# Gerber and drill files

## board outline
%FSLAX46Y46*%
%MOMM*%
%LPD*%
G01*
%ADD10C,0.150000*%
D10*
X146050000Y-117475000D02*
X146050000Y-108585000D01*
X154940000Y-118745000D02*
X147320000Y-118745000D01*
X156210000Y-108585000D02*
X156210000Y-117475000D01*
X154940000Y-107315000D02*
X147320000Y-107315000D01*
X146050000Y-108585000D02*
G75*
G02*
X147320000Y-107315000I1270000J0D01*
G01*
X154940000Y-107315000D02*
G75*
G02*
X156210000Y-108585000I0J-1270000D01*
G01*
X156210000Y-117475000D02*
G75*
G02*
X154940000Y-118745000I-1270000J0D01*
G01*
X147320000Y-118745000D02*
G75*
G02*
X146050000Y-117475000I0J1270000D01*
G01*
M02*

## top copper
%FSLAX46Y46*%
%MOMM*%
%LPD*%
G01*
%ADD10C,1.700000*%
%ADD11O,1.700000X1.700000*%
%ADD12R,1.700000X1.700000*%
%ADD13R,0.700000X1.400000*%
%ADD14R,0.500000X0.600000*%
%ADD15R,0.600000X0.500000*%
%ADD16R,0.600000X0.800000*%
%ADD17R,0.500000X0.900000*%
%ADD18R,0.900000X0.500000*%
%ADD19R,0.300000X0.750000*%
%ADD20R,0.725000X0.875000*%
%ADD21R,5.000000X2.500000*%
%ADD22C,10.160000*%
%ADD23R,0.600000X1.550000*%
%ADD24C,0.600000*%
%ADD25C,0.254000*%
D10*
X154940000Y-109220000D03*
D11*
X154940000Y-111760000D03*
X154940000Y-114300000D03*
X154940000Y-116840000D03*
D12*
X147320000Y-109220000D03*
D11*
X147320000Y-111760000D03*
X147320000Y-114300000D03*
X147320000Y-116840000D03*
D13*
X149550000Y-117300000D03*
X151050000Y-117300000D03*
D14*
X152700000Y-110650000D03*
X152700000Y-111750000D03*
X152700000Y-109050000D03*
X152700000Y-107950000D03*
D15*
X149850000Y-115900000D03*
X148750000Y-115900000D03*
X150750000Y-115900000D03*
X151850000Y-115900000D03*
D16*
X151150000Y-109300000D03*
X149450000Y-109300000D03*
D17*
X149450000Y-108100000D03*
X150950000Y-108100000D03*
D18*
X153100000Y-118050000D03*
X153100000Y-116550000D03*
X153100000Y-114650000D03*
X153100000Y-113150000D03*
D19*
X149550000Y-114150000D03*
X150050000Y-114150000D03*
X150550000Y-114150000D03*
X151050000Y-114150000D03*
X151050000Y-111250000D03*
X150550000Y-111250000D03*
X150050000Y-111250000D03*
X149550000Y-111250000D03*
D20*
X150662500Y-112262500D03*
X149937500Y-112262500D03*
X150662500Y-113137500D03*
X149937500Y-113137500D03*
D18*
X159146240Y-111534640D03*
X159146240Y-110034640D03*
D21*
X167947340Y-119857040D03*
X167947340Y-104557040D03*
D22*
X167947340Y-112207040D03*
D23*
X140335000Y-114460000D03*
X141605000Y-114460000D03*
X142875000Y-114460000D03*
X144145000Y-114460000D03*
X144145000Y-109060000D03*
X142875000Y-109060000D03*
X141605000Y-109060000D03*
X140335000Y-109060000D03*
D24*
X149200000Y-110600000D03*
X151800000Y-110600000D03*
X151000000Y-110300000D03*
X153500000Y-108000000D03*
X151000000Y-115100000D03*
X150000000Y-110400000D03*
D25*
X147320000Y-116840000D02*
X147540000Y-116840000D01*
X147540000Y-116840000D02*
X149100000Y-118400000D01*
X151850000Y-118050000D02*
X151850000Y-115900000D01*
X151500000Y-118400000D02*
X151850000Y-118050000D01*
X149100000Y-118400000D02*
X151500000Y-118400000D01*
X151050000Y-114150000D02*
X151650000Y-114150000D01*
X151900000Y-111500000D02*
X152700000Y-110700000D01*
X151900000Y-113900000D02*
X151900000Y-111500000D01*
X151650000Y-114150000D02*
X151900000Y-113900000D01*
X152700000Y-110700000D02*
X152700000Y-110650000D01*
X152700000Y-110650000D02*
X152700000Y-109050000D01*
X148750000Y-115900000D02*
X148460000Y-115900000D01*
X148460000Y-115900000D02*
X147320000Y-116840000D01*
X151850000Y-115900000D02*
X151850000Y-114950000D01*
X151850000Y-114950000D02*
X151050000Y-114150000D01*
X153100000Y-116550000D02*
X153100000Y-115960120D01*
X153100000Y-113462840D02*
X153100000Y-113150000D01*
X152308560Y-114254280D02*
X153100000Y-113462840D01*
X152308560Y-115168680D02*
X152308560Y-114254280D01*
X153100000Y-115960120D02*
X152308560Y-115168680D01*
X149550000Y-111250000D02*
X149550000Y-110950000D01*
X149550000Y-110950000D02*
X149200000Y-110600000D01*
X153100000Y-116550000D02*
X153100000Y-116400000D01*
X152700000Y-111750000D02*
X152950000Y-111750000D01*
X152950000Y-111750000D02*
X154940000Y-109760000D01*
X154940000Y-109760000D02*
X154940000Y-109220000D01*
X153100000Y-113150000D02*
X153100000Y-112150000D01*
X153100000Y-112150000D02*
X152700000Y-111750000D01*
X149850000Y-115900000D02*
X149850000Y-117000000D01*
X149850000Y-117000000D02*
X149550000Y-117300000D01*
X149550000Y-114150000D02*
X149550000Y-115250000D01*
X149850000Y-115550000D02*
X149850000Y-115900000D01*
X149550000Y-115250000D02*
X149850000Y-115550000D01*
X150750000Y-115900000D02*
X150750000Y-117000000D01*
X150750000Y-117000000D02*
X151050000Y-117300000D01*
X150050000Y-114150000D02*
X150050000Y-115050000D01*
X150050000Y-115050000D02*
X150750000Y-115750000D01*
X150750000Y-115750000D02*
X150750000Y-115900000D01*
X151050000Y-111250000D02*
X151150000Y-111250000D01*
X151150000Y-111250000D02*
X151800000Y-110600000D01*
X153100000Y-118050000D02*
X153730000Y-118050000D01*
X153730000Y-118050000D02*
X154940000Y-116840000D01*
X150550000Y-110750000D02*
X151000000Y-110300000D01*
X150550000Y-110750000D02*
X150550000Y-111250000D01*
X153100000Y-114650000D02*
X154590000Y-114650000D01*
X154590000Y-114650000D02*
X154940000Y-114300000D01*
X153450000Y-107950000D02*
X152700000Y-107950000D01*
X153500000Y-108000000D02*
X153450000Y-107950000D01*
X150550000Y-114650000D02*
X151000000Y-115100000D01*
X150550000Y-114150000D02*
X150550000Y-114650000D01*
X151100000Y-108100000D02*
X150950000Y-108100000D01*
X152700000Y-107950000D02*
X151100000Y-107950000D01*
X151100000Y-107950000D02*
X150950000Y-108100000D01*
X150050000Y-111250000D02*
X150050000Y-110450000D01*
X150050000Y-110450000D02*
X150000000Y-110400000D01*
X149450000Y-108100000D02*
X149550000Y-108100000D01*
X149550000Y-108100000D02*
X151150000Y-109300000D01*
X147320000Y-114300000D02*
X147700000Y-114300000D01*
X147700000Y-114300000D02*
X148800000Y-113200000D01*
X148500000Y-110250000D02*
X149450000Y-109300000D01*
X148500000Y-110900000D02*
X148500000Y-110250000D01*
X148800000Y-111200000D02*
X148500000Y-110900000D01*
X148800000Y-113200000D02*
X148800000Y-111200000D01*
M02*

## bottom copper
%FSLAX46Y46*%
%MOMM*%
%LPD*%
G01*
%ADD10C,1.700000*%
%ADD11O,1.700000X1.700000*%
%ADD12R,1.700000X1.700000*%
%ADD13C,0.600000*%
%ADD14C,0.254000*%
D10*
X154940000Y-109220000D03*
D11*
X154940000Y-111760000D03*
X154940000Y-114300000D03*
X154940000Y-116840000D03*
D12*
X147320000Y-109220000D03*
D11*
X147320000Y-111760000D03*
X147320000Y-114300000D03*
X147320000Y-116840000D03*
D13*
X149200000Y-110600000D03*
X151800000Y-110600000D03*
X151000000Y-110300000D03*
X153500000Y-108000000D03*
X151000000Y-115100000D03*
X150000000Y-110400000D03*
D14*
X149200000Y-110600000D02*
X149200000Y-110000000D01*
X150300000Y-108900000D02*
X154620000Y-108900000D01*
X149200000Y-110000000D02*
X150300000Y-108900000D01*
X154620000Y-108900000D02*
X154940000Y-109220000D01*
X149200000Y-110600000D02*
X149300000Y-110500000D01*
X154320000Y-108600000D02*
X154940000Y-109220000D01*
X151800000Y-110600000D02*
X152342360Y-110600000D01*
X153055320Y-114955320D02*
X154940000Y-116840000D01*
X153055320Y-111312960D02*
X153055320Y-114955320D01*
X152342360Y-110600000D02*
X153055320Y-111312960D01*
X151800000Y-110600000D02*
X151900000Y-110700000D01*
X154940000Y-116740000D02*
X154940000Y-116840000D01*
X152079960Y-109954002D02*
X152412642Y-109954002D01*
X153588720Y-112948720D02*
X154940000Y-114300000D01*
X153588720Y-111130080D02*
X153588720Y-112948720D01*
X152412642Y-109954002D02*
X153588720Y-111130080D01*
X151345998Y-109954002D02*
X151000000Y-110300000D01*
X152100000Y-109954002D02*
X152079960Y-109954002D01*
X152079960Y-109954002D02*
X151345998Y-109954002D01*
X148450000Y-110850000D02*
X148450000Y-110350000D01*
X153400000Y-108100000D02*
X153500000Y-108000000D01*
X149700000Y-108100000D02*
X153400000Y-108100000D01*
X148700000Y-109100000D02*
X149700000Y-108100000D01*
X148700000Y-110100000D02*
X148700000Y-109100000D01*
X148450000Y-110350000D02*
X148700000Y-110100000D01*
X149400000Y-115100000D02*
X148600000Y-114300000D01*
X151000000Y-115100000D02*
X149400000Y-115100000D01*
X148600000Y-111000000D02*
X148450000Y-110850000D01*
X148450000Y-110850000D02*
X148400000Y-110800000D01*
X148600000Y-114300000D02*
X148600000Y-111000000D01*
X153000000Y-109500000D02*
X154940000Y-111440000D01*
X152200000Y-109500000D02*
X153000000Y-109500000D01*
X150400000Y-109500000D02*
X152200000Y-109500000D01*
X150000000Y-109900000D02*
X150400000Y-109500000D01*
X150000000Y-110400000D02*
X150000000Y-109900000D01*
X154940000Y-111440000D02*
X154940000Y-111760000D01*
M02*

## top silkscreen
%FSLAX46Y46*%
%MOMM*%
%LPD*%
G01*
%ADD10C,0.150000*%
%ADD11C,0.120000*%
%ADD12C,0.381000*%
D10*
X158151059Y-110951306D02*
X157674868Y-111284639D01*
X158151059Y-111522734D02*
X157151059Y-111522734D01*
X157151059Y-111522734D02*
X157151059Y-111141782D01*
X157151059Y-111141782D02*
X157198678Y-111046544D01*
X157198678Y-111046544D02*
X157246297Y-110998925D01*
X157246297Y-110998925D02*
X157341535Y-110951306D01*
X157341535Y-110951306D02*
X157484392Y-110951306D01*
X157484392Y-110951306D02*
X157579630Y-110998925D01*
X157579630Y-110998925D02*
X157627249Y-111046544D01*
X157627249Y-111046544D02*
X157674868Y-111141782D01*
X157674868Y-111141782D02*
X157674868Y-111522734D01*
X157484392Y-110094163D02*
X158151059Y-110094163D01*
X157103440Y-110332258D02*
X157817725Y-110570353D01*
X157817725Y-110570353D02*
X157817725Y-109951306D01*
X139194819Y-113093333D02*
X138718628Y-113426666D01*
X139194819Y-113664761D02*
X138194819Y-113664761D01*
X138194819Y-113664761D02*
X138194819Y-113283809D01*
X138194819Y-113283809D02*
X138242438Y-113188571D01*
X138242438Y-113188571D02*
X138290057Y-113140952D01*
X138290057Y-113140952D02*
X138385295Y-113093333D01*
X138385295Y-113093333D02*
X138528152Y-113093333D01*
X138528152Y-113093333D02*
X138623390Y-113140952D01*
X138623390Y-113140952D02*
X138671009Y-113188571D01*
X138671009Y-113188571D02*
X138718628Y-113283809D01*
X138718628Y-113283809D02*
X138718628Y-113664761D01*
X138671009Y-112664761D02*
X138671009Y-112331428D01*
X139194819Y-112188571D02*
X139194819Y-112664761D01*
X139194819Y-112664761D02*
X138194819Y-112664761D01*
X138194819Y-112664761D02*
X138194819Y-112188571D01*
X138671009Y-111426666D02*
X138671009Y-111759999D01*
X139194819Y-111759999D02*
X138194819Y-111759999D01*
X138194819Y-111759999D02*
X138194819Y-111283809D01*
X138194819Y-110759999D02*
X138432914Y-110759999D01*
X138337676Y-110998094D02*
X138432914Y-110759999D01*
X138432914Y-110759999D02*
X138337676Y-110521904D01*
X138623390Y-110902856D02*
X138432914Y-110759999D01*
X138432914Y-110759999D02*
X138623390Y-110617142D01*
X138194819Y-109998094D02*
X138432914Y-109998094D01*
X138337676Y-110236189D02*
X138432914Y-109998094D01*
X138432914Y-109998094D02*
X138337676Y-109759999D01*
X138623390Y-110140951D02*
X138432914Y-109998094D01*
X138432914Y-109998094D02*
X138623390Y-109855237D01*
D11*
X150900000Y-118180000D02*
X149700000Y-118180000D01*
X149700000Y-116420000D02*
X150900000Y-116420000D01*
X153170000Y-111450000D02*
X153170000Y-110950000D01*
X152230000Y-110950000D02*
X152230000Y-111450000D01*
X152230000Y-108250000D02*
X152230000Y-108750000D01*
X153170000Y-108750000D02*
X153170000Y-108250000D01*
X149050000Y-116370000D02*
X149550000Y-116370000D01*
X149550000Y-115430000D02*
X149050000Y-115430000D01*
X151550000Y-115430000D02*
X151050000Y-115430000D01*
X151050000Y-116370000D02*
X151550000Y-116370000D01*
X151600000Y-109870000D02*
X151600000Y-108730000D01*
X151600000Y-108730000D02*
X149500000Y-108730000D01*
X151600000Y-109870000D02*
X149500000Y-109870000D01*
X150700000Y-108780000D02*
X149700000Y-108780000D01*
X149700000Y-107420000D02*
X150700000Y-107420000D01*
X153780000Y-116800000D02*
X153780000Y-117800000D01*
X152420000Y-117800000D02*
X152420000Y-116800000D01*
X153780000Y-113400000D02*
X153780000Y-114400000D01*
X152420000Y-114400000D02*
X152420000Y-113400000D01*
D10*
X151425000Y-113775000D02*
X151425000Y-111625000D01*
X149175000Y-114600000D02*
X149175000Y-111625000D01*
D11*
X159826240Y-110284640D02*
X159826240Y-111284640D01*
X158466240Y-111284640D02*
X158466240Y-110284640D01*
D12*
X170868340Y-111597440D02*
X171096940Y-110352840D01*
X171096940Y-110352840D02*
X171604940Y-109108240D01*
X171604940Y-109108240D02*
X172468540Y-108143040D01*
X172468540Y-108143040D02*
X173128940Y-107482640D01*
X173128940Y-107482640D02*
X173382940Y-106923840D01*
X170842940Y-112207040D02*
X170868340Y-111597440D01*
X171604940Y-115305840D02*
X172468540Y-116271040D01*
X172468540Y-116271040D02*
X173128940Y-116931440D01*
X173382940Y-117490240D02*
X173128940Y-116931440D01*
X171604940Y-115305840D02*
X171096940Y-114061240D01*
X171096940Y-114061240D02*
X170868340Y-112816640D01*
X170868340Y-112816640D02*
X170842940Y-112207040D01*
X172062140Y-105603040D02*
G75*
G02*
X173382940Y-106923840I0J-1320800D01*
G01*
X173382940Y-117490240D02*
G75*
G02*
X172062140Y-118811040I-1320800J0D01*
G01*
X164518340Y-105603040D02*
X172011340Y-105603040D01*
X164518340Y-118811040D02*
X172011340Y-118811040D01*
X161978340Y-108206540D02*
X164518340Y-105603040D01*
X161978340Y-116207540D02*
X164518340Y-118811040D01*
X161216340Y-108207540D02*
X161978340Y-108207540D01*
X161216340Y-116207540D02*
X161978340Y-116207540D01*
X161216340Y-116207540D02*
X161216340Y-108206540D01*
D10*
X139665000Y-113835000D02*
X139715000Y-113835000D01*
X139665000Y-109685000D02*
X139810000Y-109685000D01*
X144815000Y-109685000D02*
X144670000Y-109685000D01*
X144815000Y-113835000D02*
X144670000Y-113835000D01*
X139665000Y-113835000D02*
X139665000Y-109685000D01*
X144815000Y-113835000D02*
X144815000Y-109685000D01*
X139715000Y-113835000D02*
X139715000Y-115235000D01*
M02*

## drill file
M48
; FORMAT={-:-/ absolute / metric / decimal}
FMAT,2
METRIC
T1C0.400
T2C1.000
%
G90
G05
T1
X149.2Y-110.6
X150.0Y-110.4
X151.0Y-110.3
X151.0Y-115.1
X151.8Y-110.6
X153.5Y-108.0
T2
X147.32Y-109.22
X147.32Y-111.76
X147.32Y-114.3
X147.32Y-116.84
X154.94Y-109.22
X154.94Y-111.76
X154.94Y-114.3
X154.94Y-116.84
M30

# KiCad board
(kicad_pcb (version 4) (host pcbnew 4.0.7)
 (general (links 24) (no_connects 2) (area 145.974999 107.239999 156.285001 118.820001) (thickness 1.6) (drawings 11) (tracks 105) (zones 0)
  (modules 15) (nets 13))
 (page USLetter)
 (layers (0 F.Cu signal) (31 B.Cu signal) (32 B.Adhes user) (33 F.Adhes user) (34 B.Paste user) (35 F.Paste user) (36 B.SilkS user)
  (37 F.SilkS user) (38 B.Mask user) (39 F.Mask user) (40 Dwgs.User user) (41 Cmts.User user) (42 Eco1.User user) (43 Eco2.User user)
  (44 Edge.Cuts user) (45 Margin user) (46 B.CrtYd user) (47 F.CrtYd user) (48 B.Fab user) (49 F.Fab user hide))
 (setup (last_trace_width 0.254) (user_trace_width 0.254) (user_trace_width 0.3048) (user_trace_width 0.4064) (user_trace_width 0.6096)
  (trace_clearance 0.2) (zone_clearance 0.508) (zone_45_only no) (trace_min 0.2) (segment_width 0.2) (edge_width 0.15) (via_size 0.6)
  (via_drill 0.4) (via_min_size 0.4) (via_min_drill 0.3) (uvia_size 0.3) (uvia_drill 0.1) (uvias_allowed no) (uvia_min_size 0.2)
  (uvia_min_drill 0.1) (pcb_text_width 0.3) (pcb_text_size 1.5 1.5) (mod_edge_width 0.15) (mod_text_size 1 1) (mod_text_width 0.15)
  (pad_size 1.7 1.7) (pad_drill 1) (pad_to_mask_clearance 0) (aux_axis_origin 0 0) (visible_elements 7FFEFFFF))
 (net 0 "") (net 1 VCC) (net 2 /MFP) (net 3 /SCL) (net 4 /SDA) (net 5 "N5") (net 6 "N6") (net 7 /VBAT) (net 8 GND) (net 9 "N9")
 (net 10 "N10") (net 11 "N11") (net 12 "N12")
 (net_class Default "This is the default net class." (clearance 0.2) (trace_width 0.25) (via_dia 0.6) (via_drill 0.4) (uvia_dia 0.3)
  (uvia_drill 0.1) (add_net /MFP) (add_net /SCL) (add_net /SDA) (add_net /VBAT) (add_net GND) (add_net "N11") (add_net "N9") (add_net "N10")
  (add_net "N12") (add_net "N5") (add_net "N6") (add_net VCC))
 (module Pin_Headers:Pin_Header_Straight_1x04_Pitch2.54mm (layer F.Cu) (at 154.94 109.22)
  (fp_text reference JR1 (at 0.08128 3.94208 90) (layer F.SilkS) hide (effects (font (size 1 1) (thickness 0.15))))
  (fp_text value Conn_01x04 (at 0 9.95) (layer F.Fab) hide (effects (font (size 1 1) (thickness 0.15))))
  (pad 1 thru_hole circle (at 0 0) (size 1.7 1.7) (drill 1) (layers *.Cu *.Mask) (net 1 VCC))
  (pad 2 thru_hole oval (at 0 2.54) (size 1.7 1.7) (drill 1) (layers *.Cu *.Mask) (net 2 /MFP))
  (pad 3 thru_hole oval (at 0 5.08) (size 1.7 1.7) (drill 1) (layers *.Cu *.Mask) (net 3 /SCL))
  (pad 4 thru_hole oval (at 0 7.62) (size 1.7 1.7) (drill 1) (layers *.Cu *.Mask) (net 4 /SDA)))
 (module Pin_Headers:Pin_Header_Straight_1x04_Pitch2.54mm (layer F.Cu) (at 147.32 109.22)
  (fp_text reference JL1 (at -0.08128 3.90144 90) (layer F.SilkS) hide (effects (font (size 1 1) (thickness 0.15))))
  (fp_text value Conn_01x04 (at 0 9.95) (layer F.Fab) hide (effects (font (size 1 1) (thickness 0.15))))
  (pad 1 thru_hole rect (at 0 0) (size 1.7 1.7) (drill 1) (layers *.Cu *.Mask) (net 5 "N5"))
  (pad 2 thru_hole oval (at 0 2.54) (size 1.7 1.7) (drill 1) (layers *.Cu *.Mask) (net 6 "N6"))
  (pad 3 thru_hole oval (at 0 5.08) (size 1.7 1.7) (drill 1) (layers *.Cu *.Mask) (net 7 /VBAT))
  (pad 4 thru_hole oval (at 0 7.62) (size 1.7 1.7) (drill 1) (layers *.Cu *.Mask) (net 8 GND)))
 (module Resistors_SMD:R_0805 (layer F.Cu) (at 150.3 117.3)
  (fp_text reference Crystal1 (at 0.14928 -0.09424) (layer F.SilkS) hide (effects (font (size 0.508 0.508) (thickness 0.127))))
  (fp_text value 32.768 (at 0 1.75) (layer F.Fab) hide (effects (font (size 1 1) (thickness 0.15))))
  (fp_line (start 0.6 0.88) (end -0.6 0.88) (layer F.SilkS) (width 0.12))
  (fp_line (start -0.6 -0.88) (end 0.6 -0.88) (layer F.SilkS) (width 0.12))
  (pad 1 smd rect (at -0.75 0) (size 0.7 1.4) (layers F.Cu F.Paste F.Mask) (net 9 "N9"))
  (pad 2 smd rect (at 0.75 0) (size 0.7 1.4) (layers F.Cu F.Paste F.Mask) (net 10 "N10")))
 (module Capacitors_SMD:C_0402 (layer F.Cu) (at 152.7 111.2 270)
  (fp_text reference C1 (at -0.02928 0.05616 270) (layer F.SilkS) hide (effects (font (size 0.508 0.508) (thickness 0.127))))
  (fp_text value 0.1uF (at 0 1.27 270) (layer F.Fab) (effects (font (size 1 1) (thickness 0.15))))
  (fp_line (start 0.25 -0.47) (end -0.25 -0.47) (layer F.SilkS) (width 0.12))
  (fp_line (start -0.25 0.47) (end 0.25 0.47) (layer F.SilkS) (width 0.12))
  (pad 1 smd rect (at -0.55 0 270) (size 0.6 0.5) (layers F.Cu F.Paste F.Mask) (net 8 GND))
  (pad 2 smd rect (at 0.55 0 270) (size 0.6 0.5) (layers F.Cu F.Paste F.Mask) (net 1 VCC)))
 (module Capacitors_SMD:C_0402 (layer F.Cu) (at 152.7 108.5 90)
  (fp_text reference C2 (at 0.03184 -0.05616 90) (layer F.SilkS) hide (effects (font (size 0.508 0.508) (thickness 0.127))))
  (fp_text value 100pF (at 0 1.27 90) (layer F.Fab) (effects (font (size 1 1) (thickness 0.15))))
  (fp_line (start 0.25 -0.47) (end -0.25 -0.47) (layer F.SilkS) (width 0.12))
  (fp_line (start -0.25 0.47) (end 0.25 0.47) (layer F.SilkS) (width 0.12))
  (pad 1 smd rect (at -0.55 0 90) (size 0.6 0.5) (layers F.Cu F.Paste F.Mask) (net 8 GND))
  (pad 2 smd rect (at 0.55 0 90) (size 0.6 0.5) (layers F.Cu F.Paste F.Mask) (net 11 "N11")))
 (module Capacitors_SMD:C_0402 (layer F.Cu) (at 149.3 115.9 180)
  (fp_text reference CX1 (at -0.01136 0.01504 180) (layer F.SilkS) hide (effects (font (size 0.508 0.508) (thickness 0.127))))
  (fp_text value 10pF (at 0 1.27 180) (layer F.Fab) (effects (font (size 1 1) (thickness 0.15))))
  (fp_line (start 0.25 -0.47) (end -0.25 -0.47) (layer F.SilkS) (width 0.12))
  (fp_line (start -0.25 0.47) (end 0.25 0.47) (layer F.SilkS) (width 0.12))
  (pad 1 smd rect (at -0.55 0 180) (size 0.6 0.5) (layers F.Cu F.Paste F.Mask) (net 9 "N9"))
  (pad 2 smd rect (at 0.55 0 180) (size 0.6 0.5) (layers F.Cu F.Paste F.Mask) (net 8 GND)))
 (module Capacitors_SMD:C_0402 (layer F.Cu) (at 151.3 115.9)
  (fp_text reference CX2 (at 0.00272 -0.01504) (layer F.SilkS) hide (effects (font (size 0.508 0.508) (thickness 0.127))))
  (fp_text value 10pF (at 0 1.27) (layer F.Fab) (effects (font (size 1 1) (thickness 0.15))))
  (fp_line (start 0.25 -0.47) (end -0.25 -0.47) (layer F.SilkS) (width 0.12))
  (fp_line (start -0.25 0.47) (end 0.25 0.47) (layer F.SilkS) (width 0.12))
  (pad 1 smd rect (at -0.55 0) (size 0.6 0.5) (layers F.Cu F.Paste F.Mask) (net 10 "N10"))
  (pad 2 smd rect (at 0.55 0) (size 0.6 0.5) (layers F.Cu F.Paste F.Mask) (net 8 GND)))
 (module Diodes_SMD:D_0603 (layer F.Cu) (at 150.3 109.3 180)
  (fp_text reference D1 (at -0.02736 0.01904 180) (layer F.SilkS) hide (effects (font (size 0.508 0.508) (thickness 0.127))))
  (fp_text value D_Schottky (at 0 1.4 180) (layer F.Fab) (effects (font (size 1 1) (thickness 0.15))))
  (fp_line (start -1.3 -0.57) (end -1.3 0.57) (layer F.SilkS) (width 0.12))
  (fp_line (start -1.3 0.57) (end 0.8 0.57) (layer F.SilkS) (width 0.12))
  (fp_line (start -1.3 -0.57) (end 0.8 -0.57) (layer F.SilkS) (width 0.12))
  (pad 1 smd rect (at -0.85 0 180) (size 0.6 0.8) (layers F.Cu F.Paste F.Mask) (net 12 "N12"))
  (pad 2 smd rect (at 0.85 0 180) (size 0.6 0.8) (layers F.Cu F.Paste F.Mask) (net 7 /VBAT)))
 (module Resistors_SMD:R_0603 (layer F.Cu) (at 150.2 108.1)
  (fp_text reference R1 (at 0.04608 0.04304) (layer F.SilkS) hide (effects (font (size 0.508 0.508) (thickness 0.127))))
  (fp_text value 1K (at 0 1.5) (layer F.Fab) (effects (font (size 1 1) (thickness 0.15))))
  (fp_line (start 0.5 0.68) (end -0.5 0.68) (layer F.SilkS) (width 0.12))
  (fp_line (start -0.5 -0.68) (end 0.5 -0.68) (layer F.SilkS) (width 0.12))
  (pad 1 smd rect (at -0.75 0) (size 0.5 0.9) (layers F.Cu F.Paste F.Mask) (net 12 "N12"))
  (pad 2 smd rect (at 0.75 0) (size 0.5 0.9) (layers F.Cu F.Paste F.Mask) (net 11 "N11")))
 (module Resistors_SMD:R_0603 (layer F.Cu) (at 153.1 117.3 90)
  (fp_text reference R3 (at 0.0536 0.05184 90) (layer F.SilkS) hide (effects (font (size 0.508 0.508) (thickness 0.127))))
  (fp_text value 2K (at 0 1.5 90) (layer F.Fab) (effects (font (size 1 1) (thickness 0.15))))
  (fp_line (start 0.5 0.68) (end -0.5 0.68) (layer F.SilkS) (width 0.12))
  (fp_line (start -0.5 -0.68) (end 0.5 -0.68) (layer F.SilkS) (width 0.12))
  (pad 1 smd rect (at -0.75 0 90) (size 0.5 0.9) (layers F.Cu F.Paste F.Mask) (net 4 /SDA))
  (pad 2 smd rect (at 0.75 0 90) (size 0.5 0.9) (layers F.Cu F.Paste F.Mask) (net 1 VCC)))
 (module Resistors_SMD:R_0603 (layer F.Cu) (at 153.1 113.9 90)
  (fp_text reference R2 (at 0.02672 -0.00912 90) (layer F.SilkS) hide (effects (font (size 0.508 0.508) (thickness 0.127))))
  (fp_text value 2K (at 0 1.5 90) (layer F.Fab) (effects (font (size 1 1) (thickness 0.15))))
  (fp_line (start 0.5 0.68) (end -0.5 0.68) (layer F.SilkS) (width 0.12))
  (fp_line (start -0.5 -0.68) (end 0.5 -0.68) (layer F.SilkS) (width 0.12))
  (pad 1 smd rect (at -0.75 0 90) (size 0.5 0.9) (layers F.Cu F.Paste F.Mask) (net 3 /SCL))
  (pad 2 smd rect (at 0.75 0 90) (size 0.5 0.9) (layers F.Cu F.Paste F.Mask) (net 1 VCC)))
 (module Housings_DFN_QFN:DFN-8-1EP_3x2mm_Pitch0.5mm (layer F.Cu) (at 150.3 112.7 90)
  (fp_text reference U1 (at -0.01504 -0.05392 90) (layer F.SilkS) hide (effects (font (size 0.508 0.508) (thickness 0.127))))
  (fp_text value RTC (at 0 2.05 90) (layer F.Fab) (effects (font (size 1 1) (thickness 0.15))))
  (fp_line (start -1.075 1.125) (end 1.075 1.125) (layer F.SilkS) (width 0.15))
  (fp_line (start -1.9 -1.125) (end 1.075 -1.125) (layer F.SilkS) (width 0.15))
  (pad 1 smd rect (at -1.45 -0.75 90) (size 0.75 0.3) (layers F.Cu F.Paste F.Mask) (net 9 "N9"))
  (pad 2 smd rect (at -1.45 -0.25 90) (size 0.75 0.3) (layers F.Cu F.Paste F.Mask) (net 10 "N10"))
  (pad 3 smd rect (at -1.45 0.25 90) (size 0.75 0.3) (layers F.Cu F.Paste F.Mask) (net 11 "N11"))
  (pad 4 smd rect (at -1.45 0.75 90) (size 0.75 0.3) (layers F.Cu F.Paste F.Mask) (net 8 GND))
  (pad 5 smd rect (at 1.45 0.75 90) (size 0.75 0.3) (layers F.Cu F.Paste F.Mask) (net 4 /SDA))
  (pad 6 smd rect (at 1.45 0.25 90) (size 0.75 0.3) (layers F.Cu F.Paste F.Mask) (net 3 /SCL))
  (pad 7 smd rect (at 1.45 -0.25 90) (size 0.75 0.3) (layers F.Cu F.Paste F.Mask) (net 2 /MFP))
  (pad 8 smd rect (at 1.45 -0.75 90) (size 0.75 0.3) (layers F.Cu F.Paste F.Mask) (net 1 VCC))
  (pad 9 smd rect (at 0.4375 0.3625 90) (size 0.875 0.725) (layers F.Cu F.Paste F.Mask) (solder_paste_margin_ratio -0.2))
  (pad 9 smd rect (at 0.4375 -0.3625 90) (size 0.875 0.725) (layers F.Cu F.Paste F.Mask) (solder_paste_margin_ratio -0.2))
  (pad 9 smd rect (at -0.4375 0.3625 90) (size 0.875 0.725) (layers F.Cu F.Paste F.Mask) (solder_paste_margin_ratio -0.2))
  (pad 9 smd rect (at -0.4375 -0.3625 90) (size 0.875 0.725) (layers F.Cu F.Paste F.Mask) (solder_paste_margin_ratio -0.2)))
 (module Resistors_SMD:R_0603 (layer F.Cu) (at 159.14624 110.78464 90)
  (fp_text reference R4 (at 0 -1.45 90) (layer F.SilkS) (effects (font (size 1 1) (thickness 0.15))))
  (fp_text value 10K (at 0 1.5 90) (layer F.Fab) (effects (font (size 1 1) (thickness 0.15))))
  (fp_line (start 0.5 0.68) (end -0.5 0.68) (layer F.SilkS) (width 0.12))
  (fp_line (start -0.5 -0.68) (end 0.5 -0.68) (layer F.SilkS) (width 0.12))
  (pad 1 smd rect (at -0.75 0 90) (size 0.5 0.9) (layers F.Cu F.Paste F.Mask) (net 2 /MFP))
  (pad 2 smd rect (at 0.75 0 90) (size 0.5 0.9) (layers F.Cu F.Paste F.Mask) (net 1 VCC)))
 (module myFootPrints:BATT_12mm (layer F.Cu) (at 167.94734 112.20704 90)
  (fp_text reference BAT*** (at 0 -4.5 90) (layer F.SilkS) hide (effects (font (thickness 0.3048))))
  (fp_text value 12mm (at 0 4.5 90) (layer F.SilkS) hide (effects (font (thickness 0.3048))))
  (fp_line (start 0.6096 2.921) (end 1.8542 3.1496) (layer F.SilkS) (width 0.381))
  (fp_line (start 1.8542 3.1496) (end 3.0988 3.6576) (layer F.SilkS) (width 0.381))
  (fp_line (start 3.0988 3.6576) (end 4.064 4.5212) (layer F.SilkS) (width 0.381))
  (fp_line (start 4.064 4.5212) (end 4.7244 5.1816) (layer F.SilkS) (width 0.381))
  (fp_line (start 4.7244 5.1816) (end 5.2832 5.4356) (layer F.SilkS) (width 0.381))
  (fp_line (start 0 2.8956) (end 0.6096 2.921) (layer F.SilkS) (width 0.381))
  (fp_line (start -3.0988 3.6576) (end -4.064 4.5212) (layer F.SilkS) (width 0.381))
  (fp_line (start -4.064 4.5212) (end -4.7244 5.1816) (layer F.SilkS) (width 0.381))
  (fp_line (start -5.2832 5.4356) (end -4.7244 5.1816) (layer F.SilkS) (width 0.381))
  (fp_line (start -3.0988 3.6576) (end -1.8542 3.1496) (layer F.SilkS) (width 0.381))
  (fp_line (start -1.8542 3.1496) (end -0.6096 2.921) (layer F.SilkS) (width 0.381))
  (fp_line (start -0.6096 2.921) (end 0 2.8956) (layer F.SilkS) (width 0.381))
  (fp_arc (start 5.2832 4.1148) (end 6.604 4.1148) (angle 90) (layer F.SilkS) (width 0.381))
  (fp_arc (start -5.2832 4.1148) (end -5.2832 5.4356) (angle 90) (layer F.SilkS) (width 0.381))
  (fp_line (start 6.604 -3.429) (end 6.604 4.064) (layer F.SilkS) (width 0.381))
  (fp_line (start -6.604 -3.429) (end -6.604 4.064) (layer F.SilkS) (width 0.381))
  (fp_line (start 4.0005 -5.969) (end 6.604 -3.429) (layer F.SilkS) (width 0.381))
  (fp_line (start -4.0005 -5.969) (end -6.604 -3.429) (layer F.SilkS) (width 0.381))
  (fp_line (start 3.9995 -6.731) (end 3.9995 -5.969) (layer F.SilkS) (width 0.381))
  (fp_line (start -4.0005 -6.731) (end -4.0005 -5.969) (layer F.SilkS) (width 0.381))
  (fp_line (start -4.0005 -6.731) (end 4.0005 -6.731) (layer F.SilkS) (width 0.381))
  (pad 1 smd rect (at -7.65 0 90) (size 2.5 5) (layers F.Cu F.Paste F.Mask))
  (pad 1 smd rect (at 7.65 0 90) (size 2.5 5) (layers F.Cu F.Paste F.Mask))
  (pad 2 smd circle (at 0 0 90) (size 10.16 10.16) (layers F.Cu F.Paste F.Mask)))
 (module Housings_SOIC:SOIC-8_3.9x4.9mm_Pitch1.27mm (layer F.Cu) (at 142.24 111.76 90)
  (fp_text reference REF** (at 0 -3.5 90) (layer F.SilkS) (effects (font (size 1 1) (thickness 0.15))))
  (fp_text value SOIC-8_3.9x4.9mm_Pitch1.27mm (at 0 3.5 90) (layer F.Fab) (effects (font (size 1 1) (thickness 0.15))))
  (fp_line (start -2.075 -2.575) (end -2.075 -2.525) (layer F.SilkS) (width 0.15))
  (fp_line (start 2.075 -2.575) (end 2.075 -2.43) (layer F.SilkS) (width 0.15))
  (fp_line (start 2.075 2.575) (end 2.075 2.43) (layer F.SilkS) (width 0.15))
  (fp_line (start -2.075 2.575) (end -2.075 2.43) (layer F.SilkS) (width 0.15))
  (fp_line (start -2.075 -2.575) (end 2.075 -2.575) (layer F.SilkS) (width 0.15))
  (fp_line (start -2.075 2.575) (end 2.075 2.575) (layer F.SilkS) (width 0.15))
  (fp_line (start -2.075 -2.525) (end -3.475 -2.525) (layer F.SilkS) (width 0.15))
  (pad 1 smd rect (at -2.7 -1.905 90) (size 1.55 0.6) (layers F.Cu F.Paste F.Mask))
  (pad 2 smd rect (at -2.7 -0.635 90) (size 1.55 0.6) (layers F.Cu F.Paste F.Mask))
  (pad 3 smd rect (at -2.7 0.635 90) (size 1.55 0.6) (layers F.Cu F.Paste F.Mask))
  (pad 4 smd rect (at -2.7 1.905 90) (size 1.55 0.6) (layers F.Cu F.Paste F.Mask))
  (pad 5 smd rect (at 2.7 1.905 90) (size 1.55 0.6) (layers F.Cu F.Paste F.Mask))
  (pad 6 smd rect (at 2.7 0.635 90) (size 1.55 0.6) (layers F.Cu F.Paste F.Mask))
  (pad 7 smd rect (at 2.7 -0.635 90) (size 1.55 0.6) (layers F.Cu F.Paste F.Mask))
  (pad 8 smd rect (at 2.7 -1.905 90) (size 1.55 0.6) (layers F.Cu F.Paste F.Mask)))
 (gr_line (start 146.05 117.475) (end 146.05 108.585) (angle 90) (layer Edge.Cuts) (width 0.15))
 (gr_line (start 154.94 118.745) (end 147.32 118.745) (angle 90) (layer Edge.Cuts) (width 0.15))
 (gr_line (start 156.21 108.585) (end 156.21 117.475) (angle 90) (layer Edge.Cuts) (width 0.15))
 (gr_line (start 154.94 107.315) (end 147.32 107.315) (angle 90) (layer Edge.Cuts) (width 0.15))
 (gr_arc (start 147.32 108.585) (end 146.05 108.585) (angle 90) (layer Edge.Cuts) (width 0.15))
 (gr_arc (start 154.94 108.585) (end 154.94 107.315) (angle 90) (layer Edge.Cuts) (width 0.15))
 (gr_arc (start 154.94 117.475) (end 156.21 117.475) (angle 90) (layer Edge.Cuts) (width 0.15))
 (gr_arc (start 147.32 117.475) (end 147.32 118.745) (angle 90) (layer Edge.Cuts) (width 0.15))
 (segment (start 147.32 116.84) (end 147.54 116.84) (width 0.254) (layer F.Cu) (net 8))
 (segment (start 147.54 116.84) (end 149.1 118.4) (width 0.254) (layer F.Cu) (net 8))
 (segment (start 151.85 118.05) (end 151.85 115.9) (width 0.254) (layer F.Cu) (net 8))
 (segment (start 151.5 118.4) (end 151.85 118.05) (width 0.254) (layer F.Cu) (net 8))
 (segment (start 149.1 118.4) (end 151.5 118.4) (width 0.254) (layer F.Cu) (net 8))
 (segment (start 151.05 114.15) (end 151.65 114.15) (width 0.254) (layer F.Cu) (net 8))
 (segment (start 151.9 111.5) (end 152.7 110.7) (width 0.254) (layer F.Cu) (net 8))
 (segment (start 151.9 113.9) (end 151.9 111.5) (width 0.254) (layer F.Cu) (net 8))
 (segment (start 151.65 114.15) (end 151.9 113.9) (width 0.254) (layer F.Cu) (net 8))
 (segment (start 152.7 110.7) (end 152.7 110.65) (width 0.254) (layer F.Cu) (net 8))
 (segment (start 152.7 110.65) (end 152.7 109.05) (width 0.254) (layer F.Cu) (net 8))
 (segment (start 148.75 115.9) (end 148.46 115.9) (width 0.254) (layer F.Cu) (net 8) (status 30))
 (segment (start 148.46 115.9) (end 147.32 116.84) (width 0.254) (layer F.Cu) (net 8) (status 10))
 (segment (start 151.85 115.9) (end 151.85 114.95) (width 0.254) (layer F.Cu) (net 8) (status 10))
 (segment (start 151.85 114.95) (end 151.05 114.15) (width 0.254) (layer F.Cu) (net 8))
 (segment (start 153.1 116.55) (end 153.1 115.96012) (width 0.254) (layer F.Cu) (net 1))
 (segment (start 153.1 113.46284) (end 153.1 113.15) (width 0.254) (layer F.Cu) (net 1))
 (segment (start 152.30856 114.25428) (end 153.1 113.46284) (width 0.254) (layer F.Cu) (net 1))
 (segment (start 152.30856 115.16868) (end 152.30856 114.25428) (width 0.254) (layer F.Cu) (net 1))
 (segment (start 153.1 115.96012) (end 152.30856 115.16868) (width 0.254) (layer F.Cu) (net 1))
 (segment (start 149.2 110.6) (end 149.2 110) (width 0.254) (layer B.Cu) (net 1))
 (segment (start 150.3 108.9) (end 154.62 108.9) (width 0.254) (layer B.Cu) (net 1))
 (segment (start 149.2 110) (end 150.3 108.9) (width 0.254) (layer B.Cu) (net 1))
 (segment (start 154.62 108.9) (end 154.94 109.22) (width 0.254) (layer B.Cu) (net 1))
 (segment (start 149.55 111.25) (end 149.55 110.95) (width 0.254) (layer F.Cu) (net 1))
 (segment (start 149.55 110.95) (end 149.2 110.6) (width 0.254) (layer F.Cu) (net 1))
 (via (at 149.2 110.6) (size 0.6) (drill 0.4) (layers F.Cu B.Cu) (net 1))
 (segment (start 149.2 110.6) (end 149.3 110.5) (width 0.254) (layer B.Cu) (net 1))
 (segment (start 154.32 108.6) (end 154.94 109.22) (width 0.254) (layer B.Cu) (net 1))
 (segment (start 153.1 116.55) (end 153.1 116.4) (width 0.254) (layer F.Cu) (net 1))
 (segment (start 152.7 111.75) (end 152.95 111.75) (width 0.254) (layer F.Cu) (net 1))
 (segment (start 152.95 111.75) (end 154.94 109.76) (width 0.254) (layer F.Cu) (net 1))
 (segment (start 154.94 109.76) (end 154.94 109.22) (width 0.254) (layer F.Cu) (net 1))
 (segment (start 153.1 113.15) (end 153.1 112.15) (width 0.254) (layer F.Cu) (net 1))
 (segment (start 153.1 112.15) (end 152.7 111.75) (width 0.254) (layer F.Cu) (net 1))
 (segment (start 149.85 115.9) (end 149.85 117) (width 0.254) (layer F.Cu) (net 9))
 (segment (start 149.85 117) (end 149.55 117.3) (width 0.254) (layer F.Cu) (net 9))
 (segment (start 149.55 114.15) (end 149.55 115.25) (width 0.254) (layer F.Cu) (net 9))
 (segment (start 149.85 115.55) (end 149.85 115.9) (width 0.254) (layer F.Cu) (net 9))
 (segment (start 149.55 115.25) (end 149.85 115.55) (width 0.254) (layer F.Cu) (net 9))
 (segment (start 150.75 115.9) (end 150.75 117) (width 0.254) (layer F.Cu) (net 10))
 (segment (start 150.75 117) (end 151.05 117.3) (width 0.254) (layer F.Cu) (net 10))
 (segment (start 150.05 114.15) (end 150.05 115.05) (width 0.254) (layer F.Cu) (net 10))
 (segment (start 150.05 115.05) (end 150.75 115.75) (width 0.254) (layer F.Cu) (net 10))
 (segment (start 150.75 115.75) (end 150.75 115.9) (width 0.254) (layer F.Cu) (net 10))
 (segment (start 151.8 110.6) (end 152.34236 110.6) (width 0.254) (layer B.Cu) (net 4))
 (segment (start 153.05532 114.95532) (end 154.94 116.84) (width 0.254) (layer B.Cu) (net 4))
 (segment (start 153.05532 111.31296) (end 153.05532 114.95532) (width 0.254) (layer B.Cu) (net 4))
 (segment (start 152.34236 110.6) (end 153.05532 111.31296) (width 0.254) (layer B.Cu) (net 4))
 (segment (start 151.05 111.25) (end 151.15 111.25) (width 0.254) (layer F.Cu) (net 4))
 (segment (start 151.15 111.25) (end 151.8 110.6) (width 0.254) (layer F.Cu) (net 4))
 (via (at 151.8 110.6) (size 0.6) (drill 0.4) (layers F.Cu B.Cu) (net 4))
 (segment (start 151.8 110.6) (end 151.9 110.7) (width 0.254) (layer B.Cu) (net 4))
 (segment (start 154.94 116.74) (end 154.94 116.84) (width 0.254) (layer B.Cu) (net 4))
 (segment (start 153.1 118.05) (end 153.73 118.05) (width 0.254) (layer F.Cu) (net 4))
 (segment (start 153.73 118.05) (end 154.94 116.84) (width 0.254) (layer F.Cu) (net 4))
 (segment (start 152.07996 109.954002) (end 152.412642 109.954002) (width 0.254) (layer B.Cu) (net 3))
 (segment (start 153.58872 112.94872) (end 154.94 114.3) (width 0.254) (layer B.Cu) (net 3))
 (segment (start 153.58872 111.13008) (end 153.58872 112.94872) (width 0.254) (layer B.Cu) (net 3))
 (segment (start 152.412642 109.954002) (end 153.58872 111.13008) (width 0.254) (layer B.Cu) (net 3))
 (segment (start 150.55 110.75) (end 151 110.3) (width 0.254) (layer F.Cu) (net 3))
 (via (at 151 110.3) (size 0.6) (drill 0.4) (layers F.Cu B.Cu) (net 3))
 (segment (start 150.55 110.75) (end 150.55 111.25) (width 0.254) (layer F.Cu) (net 3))
 (segment (start 151.345998 109.954002) (end 151 110.3) (width 0.254) (layer B.Cu) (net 3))
 (segment (start 152.1 109.954002) (end 152.07996 109.954002) (width 0.254) (layer B.Cu) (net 3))
 (segment (start 152.07996 109.954002) (end 151.345998 109.954002) (width 0.254) (layer B.Cu) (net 3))
 (segment (start 153.1 114.65) (end 154.59 114.65) (width 0.254) (layer F.Cu) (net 3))
 (segment (start 154.59 114.65) (end 154.94 114.3) (width 0.254) (layer F.Cu) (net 3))
 (segment (start 148.45 110.85) (end 148.45 110.35) (width 0.254) (layer B.Cu) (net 11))
 (segment (start 153.45 107.95) (end 152.7 107.95) (width 0.254) (layer F.Cu) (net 11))
 (segment (start 153.5 108) (end 153.45 107.95) (width 0.254) (layer F.Cu) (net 11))
 (via (at 153.5 108) (size 0.6) (drill 0.4) (layers F.Cu B.Cu) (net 11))
 (segment (start 153.4 108.1) (end 153.5 108) (width 0.254) (layer B.Cu) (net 11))
 (segment (start 149.7 108.1) (end 153.4 108.1) (width 0.254) (layer B.Cu) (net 11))
 (segment (start 148.7 109.1) (end 149.7 108.1) (width 0.254) (layer B.Cu) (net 11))
 (segment (start 148.7 110.1) (end 148.7 109.1) (width 0.254) (layer B.Cu) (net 11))
 (segment (start 148.45 110.35) (end 148.7 110.1) (width 0.254) (layer B.Cu) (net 11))
 (segment (start 149.4 115.1) (end 148.6 114.3) (width 0.254) (layer B.Cu) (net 11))
 (segment (start 151 115.1) (end 149.4 115.1) (width 0.254) (layer B.Cu) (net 11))
 (via (at 151 115.1) (size 0.6) (drill 0.4) (layers F.Cu B.Cu) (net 11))
 (segment (start 150.55 114.65) (end 151 115.1) (width 0.254) (layer F.Cu) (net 11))
 (segment (start 150.55 114.15) (end 150.55 114.65) (width 0.254) (layer F.Cu) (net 11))
 (segment (start 148.6 111) (end 148.45 110.85) (width 0.254) (layer B.Cu) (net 11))
 (segment (start 148.45 110.85) (end 148.4 110.8) (width 0.254) (layer B.Cu) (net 11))
 (segment (start 148.6 114.3) (end 148.6 111) (width 0.254) (layer B.Cu) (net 11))
 (segment (start 151.1 108.1) (end 150.95 108.1) (width 0.254) (layer F.Cu) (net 11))
 (segment (start 152.7 107.95) (end 151.1 107.95) (width 0.254) (layer F.Cu) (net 11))
 (segment (start 151.1 107.95) (end 150.95 108.1) (width 0.254) (layer F.Cu) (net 11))
 (segment (start 150.05 111.25) (end 150.05 110.45) (width 0.254) (layer F.Cu) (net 2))
 (segment (start 153 109.5) (end 154.94 111.44) (width 0.254) (layer B.Cu) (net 2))
 (segment (start 152.2 109.5) (end 153 109.5) (width 0.254) (layer B.Cu) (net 2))
 (segment (start 150.4 109.5) (end 152.2 109.5) (width 0.254) (layer B.Cu) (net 2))
 (segment (start 150 109.9) (end 150.4 109.5) (width 0.254) (layer B.Cu) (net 2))
 (segment (start 150 110.4) (end 150 109.9) (width 0.254) (layer B.Cu) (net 2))
 (via (at 150 110.4) (size 0.6) (drill 0.4) (layers F.Cu B.Cu) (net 2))
 (segment (start 150.05 110.45) (end 150 110.4) (width 0.254) (layer F.Cu) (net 2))
 (segment (start 154.94 111.44) (end 154.94 111.76) (width 0.254) (layer B.Cu) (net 2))
 (segment (start 149.45 108.1) (end 149.55 108.1) (width 0.254) (layer F.Cu) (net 12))
 (segment (start 149.55 108.1) (end 151.15 109.3) (width 0.254) (layer F.Cu) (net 12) (status 20))
 (segment (start 147.32 114.3) (end 147.7 114.3) (width 0.254) (layer F.Cu) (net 7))
 (segment (start 147.7 114.3) (end 148.8 113.2) (width 0.254) (layer F.Cu) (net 7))
 (segment (start 148.5 110.25) (end 149.45 109.3) (width 0.254) (layer F.Cu) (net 7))
 (segment (start 148.5 110.9) (end 148.5 110.25) (width 0.254) (layer F.Cu) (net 7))
 (segment (start 148.8 111.2) (end 148.5 110.9) (width 0.254) (layer F.Cu) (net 7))
 (segment (start 148.8 113.2) (end 148.8 111.2) (width 0.254) (layer F.Cu) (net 7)))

